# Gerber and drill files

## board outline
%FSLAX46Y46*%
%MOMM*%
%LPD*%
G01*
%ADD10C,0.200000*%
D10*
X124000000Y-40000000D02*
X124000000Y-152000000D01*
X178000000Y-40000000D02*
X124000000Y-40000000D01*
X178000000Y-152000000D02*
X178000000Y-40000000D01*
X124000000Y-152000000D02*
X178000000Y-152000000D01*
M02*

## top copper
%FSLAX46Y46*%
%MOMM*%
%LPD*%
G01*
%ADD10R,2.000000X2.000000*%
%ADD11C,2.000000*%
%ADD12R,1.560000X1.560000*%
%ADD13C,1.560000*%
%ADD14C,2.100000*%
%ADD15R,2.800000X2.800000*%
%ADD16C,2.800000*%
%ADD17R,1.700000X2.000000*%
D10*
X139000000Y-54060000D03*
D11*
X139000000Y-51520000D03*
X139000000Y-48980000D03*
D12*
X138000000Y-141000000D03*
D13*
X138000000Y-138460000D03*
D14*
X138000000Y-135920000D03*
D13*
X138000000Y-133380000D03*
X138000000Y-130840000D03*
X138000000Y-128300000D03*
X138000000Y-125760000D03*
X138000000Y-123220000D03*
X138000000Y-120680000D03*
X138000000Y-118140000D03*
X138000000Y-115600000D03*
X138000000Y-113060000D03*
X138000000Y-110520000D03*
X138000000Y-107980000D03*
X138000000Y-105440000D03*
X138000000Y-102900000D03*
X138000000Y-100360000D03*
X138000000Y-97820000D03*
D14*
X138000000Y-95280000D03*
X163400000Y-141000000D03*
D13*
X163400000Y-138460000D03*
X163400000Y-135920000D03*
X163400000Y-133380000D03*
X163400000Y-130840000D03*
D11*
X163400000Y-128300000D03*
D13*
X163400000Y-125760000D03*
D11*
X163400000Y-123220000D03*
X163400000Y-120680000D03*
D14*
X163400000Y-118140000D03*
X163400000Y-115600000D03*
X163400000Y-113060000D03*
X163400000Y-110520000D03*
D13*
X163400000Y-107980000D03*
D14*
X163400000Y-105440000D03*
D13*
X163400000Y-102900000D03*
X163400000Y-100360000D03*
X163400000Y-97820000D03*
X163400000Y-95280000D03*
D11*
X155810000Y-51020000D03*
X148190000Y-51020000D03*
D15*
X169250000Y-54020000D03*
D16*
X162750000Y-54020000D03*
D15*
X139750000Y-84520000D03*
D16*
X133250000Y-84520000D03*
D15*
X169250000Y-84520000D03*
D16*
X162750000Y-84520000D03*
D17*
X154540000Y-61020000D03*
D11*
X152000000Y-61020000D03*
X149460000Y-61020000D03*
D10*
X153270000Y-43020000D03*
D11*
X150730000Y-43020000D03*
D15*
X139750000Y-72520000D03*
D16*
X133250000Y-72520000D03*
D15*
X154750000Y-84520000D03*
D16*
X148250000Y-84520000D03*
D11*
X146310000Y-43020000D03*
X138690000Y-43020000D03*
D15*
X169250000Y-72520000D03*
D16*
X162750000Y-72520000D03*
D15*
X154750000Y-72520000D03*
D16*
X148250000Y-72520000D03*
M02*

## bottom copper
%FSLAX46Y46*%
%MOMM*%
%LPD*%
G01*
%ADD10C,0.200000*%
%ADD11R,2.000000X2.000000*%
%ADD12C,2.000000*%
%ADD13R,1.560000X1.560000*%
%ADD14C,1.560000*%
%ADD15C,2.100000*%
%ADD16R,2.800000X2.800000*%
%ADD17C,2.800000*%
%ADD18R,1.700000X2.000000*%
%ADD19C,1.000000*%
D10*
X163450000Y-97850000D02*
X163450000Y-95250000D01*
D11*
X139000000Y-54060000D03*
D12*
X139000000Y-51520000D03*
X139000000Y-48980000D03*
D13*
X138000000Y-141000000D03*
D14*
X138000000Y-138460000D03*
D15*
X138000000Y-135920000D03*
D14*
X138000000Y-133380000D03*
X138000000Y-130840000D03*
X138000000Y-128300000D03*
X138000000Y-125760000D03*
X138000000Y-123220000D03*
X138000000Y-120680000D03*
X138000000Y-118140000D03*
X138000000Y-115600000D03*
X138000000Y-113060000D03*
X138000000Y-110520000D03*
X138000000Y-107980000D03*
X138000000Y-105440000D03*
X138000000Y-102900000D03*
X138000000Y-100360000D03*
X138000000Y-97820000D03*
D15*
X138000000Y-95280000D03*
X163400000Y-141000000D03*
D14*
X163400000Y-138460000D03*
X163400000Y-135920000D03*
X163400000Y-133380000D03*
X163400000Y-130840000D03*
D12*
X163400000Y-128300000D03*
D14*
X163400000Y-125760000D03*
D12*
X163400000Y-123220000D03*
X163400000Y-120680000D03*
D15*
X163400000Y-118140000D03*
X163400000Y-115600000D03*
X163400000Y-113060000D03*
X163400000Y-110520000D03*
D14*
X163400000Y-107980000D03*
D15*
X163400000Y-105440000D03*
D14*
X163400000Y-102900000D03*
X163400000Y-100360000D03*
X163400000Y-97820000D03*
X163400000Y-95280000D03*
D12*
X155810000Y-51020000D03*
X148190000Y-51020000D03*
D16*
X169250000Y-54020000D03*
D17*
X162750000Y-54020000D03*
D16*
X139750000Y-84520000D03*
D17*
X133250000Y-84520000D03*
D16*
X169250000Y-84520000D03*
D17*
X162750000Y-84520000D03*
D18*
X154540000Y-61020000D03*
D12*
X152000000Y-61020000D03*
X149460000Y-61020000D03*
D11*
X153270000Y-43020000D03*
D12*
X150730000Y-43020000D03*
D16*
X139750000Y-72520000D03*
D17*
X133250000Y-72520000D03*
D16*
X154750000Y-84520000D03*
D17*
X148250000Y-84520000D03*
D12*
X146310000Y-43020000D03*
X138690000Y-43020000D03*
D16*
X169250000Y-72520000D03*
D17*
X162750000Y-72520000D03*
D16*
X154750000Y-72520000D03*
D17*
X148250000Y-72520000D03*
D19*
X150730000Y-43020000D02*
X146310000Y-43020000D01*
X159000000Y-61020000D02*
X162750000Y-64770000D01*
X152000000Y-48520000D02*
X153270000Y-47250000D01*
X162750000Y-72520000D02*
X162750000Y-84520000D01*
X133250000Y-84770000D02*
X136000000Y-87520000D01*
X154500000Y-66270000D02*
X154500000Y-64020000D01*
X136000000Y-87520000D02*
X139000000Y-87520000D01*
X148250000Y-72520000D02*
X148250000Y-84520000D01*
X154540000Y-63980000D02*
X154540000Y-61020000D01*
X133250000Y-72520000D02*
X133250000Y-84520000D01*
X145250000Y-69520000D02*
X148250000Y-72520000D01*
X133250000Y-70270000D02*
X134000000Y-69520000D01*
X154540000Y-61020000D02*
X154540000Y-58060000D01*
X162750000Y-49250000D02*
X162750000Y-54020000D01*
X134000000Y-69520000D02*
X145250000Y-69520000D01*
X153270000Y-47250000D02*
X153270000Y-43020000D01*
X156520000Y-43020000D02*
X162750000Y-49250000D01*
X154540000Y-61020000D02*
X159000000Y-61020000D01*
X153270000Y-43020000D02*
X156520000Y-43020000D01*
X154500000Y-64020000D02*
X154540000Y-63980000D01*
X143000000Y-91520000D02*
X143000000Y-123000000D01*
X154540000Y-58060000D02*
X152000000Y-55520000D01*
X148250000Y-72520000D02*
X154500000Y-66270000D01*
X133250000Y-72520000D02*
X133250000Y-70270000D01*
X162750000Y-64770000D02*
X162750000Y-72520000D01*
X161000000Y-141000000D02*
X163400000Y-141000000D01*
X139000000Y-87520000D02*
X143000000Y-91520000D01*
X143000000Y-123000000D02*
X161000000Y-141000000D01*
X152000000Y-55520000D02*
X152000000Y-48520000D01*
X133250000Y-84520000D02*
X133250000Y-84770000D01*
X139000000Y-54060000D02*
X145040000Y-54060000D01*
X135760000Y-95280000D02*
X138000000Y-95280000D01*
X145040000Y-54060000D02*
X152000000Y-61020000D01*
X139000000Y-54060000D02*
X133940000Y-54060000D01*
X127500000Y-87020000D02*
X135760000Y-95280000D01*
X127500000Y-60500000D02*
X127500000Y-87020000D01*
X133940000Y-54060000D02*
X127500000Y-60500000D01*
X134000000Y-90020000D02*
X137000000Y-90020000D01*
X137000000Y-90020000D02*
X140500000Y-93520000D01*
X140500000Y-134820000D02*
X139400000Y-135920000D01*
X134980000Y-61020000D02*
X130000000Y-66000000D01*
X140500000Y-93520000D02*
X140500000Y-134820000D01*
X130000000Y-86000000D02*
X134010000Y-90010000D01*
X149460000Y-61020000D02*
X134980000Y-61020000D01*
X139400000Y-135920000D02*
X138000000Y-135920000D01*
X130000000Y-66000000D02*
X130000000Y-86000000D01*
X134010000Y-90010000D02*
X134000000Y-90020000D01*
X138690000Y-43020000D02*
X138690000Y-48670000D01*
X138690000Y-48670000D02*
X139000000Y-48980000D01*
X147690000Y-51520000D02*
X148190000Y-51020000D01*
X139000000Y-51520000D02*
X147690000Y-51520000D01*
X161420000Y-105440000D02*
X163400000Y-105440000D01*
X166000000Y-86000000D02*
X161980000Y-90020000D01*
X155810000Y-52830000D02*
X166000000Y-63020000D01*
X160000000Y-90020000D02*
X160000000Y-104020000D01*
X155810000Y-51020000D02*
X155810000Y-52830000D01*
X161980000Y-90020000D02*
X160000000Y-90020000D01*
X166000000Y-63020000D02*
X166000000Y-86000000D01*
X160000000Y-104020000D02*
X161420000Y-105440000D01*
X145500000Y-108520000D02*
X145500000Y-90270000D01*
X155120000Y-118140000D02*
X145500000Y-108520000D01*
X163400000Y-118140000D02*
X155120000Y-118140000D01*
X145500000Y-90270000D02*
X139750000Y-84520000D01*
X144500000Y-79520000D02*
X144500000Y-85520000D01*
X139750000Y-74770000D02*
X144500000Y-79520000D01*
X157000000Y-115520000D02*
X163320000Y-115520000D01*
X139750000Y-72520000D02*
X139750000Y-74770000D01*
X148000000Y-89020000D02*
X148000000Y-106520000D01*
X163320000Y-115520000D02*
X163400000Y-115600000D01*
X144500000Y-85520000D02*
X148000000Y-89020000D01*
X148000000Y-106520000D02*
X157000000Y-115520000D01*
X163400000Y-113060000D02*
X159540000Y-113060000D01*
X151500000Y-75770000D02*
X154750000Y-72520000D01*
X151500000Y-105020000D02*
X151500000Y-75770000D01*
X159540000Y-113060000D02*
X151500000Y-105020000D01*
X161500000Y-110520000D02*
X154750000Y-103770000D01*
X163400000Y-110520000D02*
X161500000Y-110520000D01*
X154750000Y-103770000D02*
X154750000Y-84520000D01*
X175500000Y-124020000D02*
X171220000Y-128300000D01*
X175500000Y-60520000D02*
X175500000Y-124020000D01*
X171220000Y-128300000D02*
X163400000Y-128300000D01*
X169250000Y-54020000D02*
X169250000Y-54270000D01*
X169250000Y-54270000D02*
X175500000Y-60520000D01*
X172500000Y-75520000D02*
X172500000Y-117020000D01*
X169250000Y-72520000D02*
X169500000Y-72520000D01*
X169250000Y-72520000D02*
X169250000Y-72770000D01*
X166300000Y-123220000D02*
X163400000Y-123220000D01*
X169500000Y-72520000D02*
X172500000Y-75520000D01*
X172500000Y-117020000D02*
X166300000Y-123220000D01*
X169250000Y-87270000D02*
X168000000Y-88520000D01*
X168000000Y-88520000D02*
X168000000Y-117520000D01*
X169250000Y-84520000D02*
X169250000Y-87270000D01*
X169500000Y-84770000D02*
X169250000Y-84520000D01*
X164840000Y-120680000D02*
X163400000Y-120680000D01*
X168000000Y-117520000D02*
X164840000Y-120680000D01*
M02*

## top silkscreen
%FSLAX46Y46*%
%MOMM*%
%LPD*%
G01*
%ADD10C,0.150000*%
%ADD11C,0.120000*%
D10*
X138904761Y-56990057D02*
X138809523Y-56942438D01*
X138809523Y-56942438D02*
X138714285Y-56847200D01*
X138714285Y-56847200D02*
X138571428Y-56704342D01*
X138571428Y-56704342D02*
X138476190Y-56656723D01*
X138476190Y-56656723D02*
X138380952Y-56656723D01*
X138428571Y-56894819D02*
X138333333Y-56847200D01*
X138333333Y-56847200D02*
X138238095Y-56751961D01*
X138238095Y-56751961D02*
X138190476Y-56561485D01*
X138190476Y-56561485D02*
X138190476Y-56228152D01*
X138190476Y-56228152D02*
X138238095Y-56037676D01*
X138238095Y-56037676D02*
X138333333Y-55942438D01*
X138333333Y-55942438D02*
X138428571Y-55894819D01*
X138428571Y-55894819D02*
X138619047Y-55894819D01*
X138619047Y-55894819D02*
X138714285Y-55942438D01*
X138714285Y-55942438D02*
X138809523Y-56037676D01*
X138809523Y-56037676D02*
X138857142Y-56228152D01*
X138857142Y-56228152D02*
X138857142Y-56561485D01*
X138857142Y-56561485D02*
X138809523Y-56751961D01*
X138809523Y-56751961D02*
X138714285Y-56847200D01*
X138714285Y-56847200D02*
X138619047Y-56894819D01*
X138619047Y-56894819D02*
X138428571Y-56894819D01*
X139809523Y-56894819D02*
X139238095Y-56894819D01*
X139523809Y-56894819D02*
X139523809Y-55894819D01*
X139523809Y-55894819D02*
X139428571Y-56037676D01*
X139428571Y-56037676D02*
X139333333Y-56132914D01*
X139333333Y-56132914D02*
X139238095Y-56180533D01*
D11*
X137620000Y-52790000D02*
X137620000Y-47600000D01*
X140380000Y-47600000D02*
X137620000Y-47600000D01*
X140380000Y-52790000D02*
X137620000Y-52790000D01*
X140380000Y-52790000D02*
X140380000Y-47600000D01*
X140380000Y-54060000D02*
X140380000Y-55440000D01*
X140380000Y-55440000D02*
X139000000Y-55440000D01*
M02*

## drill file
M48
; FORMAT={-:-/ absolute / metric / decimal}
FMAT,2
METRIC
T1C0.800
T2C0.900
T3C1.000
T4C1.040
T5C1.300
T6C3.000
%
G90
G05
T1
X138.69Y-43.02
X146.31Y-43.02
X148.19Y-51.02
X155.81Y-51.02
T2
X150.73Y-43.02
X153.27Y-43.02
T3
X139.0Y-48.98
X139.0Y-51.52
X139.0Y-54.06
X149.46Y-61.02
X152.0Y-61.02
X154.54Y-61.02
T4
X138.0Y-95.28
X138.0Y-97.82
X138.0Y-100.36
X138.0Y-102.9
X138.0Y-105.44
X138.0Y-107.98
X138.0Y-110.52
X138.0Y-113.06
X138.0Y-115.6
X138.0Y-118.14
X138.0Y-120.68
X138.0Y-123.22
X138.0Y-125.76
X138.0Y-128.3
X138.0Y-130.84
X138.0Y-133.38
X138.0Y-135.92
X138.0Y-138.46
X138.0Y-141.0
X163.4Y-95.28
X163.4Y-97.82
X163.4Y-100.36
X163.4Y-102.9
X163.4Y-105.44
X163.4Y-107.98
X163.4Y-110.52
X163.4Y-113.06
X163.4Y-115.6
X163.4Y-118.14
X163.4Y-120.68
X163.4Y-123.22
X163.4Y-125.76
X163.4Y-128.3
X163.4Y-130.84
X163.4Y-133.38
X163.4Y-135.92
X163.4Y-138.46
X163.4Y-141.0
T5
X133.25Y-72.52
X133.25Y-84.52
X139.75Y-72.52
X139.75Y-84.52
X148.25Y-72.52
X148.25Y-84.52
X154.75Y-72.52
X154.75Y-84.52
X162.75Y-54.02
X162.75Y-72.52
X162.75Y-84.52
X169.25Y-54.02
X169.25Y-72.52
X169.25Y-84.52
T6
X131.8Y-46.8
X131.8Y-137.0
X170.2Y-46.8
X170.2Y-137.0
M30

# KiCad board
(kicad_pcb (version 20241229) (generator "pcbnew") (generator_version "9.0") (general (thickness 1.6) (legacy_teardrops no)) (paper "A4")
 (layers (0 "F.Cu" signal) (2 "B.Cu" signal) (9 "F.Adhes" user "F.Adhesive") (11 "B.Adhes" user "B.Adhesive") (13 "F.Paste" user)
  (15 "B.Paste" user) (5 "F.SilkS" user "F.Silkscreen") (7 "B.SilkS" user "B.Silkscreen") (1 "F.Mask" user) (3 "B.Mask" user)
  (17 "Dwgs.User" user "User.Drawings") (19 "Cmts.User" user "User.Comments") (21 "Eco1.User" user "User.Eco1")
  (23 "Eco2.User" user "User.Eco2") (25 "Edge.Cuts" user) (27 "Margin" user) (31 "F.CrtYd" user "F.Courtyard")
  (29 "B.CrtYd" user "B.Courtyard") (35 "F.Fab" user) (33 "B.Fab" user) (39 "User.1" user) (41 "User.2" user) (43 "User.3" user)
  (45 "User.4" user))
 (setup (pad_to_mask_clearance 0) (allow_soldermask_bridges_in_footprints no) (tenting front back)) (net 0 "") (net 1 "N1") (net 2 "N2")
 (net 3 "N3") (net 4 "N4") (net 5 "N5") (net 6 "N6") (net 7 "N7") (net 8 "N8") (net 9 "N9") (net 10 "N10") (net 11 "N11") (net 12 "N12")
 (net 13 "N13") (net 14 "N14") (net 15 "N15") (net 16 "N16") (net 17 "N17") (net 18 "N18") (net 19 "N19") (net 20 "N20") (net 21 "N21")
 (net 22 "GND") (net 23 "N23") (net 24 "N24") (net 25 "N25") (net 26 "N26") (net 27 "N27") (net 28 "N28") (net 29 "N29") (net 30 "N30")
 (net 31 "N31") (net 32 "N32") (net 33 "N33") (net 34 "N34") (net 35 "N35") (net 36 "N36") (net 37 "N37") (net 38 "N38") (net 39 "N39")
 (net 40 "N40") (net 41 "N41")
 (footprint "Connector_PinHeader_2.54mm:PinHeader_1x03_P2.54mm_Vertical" (layer "F.Cu") (at 139 54.06 180)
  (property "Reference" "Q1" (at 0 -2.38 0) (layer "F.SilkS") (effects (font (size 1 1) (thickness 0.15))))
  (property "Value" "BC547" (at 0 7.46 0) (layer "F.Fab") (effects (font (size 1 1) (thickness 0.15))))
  (fp_line (start 1.38 1.27) (end 1.38 6.46) (stroke (width 0.12) (type solid)) (layer "F.SilkS"))
  (fp_line (start -1.38 6.46) (end 1.38 6.46) (stroke (width 0.12) (type solid)) (layer "F.SilkS"))
  (fp_line (start -1.38 1.27) (end 1.38 1.27) (stroke (width 0.12) (type solid)) (layer "F.SilkS"))
  (fp_line (start -1.38 1.27) (end -1.38 6.46) (stroke (width 0.12) (type solid)) (layer "F.SilkS"))
  (fp_line (start -1.38 0) (end -1.38 -1.38) (stroke (width 0.12) (type solid)) (layer "F.SilkS"))
  (fp_line (start -1.38 -1.38) (end 0 -1.38) (stroke (width 0.12) (type solid)) (layer "F.SilkS"))
  (pad "1" thru_hole rect (at 0 0 180) (size 2 2) (drill 1) (layers "*.Cu" "*.Mask") (remove_unused_layers no) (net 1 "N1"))
  (pad "2" thru_hole circle (at 0 2.54 180) (size 2 2) (drill 1) (layers "*.Cu" "*.Mask") (remove_unused_layers no) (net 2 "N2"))
  (pad "3" thru_hole circle (at 0 5.08 180) (size 2 2) (drill 1) (layers "*.Cu" "*.Mask") (remove_unused_layers no) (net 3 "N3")))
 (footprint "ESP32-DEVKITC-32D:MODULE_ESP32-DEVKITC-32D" (layer "B.Cu") (at 150.7 121.24)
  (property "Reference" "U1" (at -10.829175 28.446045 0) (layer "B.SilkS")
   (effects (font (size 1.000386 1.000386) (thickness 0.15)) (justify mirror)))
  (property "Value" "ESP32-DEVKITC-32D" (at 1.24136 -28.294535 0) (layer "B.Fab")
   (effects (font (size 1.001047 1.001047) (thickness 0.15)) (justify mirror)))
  (pad "J2-1" thru_hole rect (at -12.7 19.76) (size 1.56 1.56) (drill 1.04) (layers "*.Cu" "*.Mask") (remove_unused_layers no) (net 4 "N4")
   (solder_mask_margin 0.102))
  (pad "J2-2" thru_hole circle (at -12.7 17.22) (size 1.56 1.56) (drill 1.04) (layers "*.Cu" "*.Mask") (remove_unused_layers no)
   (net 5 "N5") (solder_mask_margin 0.102))
  (pad "J2-3" thru_hole circle (at -12.7 14.68) (size 2.1 2.1) (drill 1.04) (layers "*.Cu" "*.Mask") (remove_unused_layers no) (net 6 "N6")
   (solder_mask_margin 0.102))
  (pad "J2-4" thru_hole circle (at -12.7 12.14) (size 1.56 1.56) (drill 1.04) (layers "*.Cu" "*.Mask") (remove_unused_layers no)
   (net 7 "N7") (solder_mask_margin 0.102))
  (pad "J2-5" thru_hole circle (at -12.7 9.6) (size 1.56 1.56) (drill 1.04) (layers "*.Cu" "*.Mask") (remove_unused_layers no) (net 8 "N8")
   (solder_mask_margin 0.102))
  (pad "J2-6" thru_hole circle (at -12.7 7.06) (size 1.56 1.56) (drill 1.04) (layers "*.Cu" "*.Mask") (remove_unused_layers no) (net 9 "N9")
   (solder_mask_margin 0.102))
  (pad "J2-7" thru_hole circle (at -12.7 4.52) (size 1.56 1.56) (drill 1.04) (layers "*.Cu" "*.Mask") (remove_unused_layers no)
   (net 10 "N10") (solder_mask_margin 0.102))
  (pad "J2-8" thru_hole circle (at -12.7 1.98) (size 1.56 1.56) (drill 1.04) (layers "*.Cu" "*.Mask") (remove_unused_layers no)
   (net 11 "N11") (solder_mask_margin 0.102))
  (pad "J2-9" thru_hole circle (at -12.7 -0.56) (size 1.56 1.56) (drill 1.04) (layers "*.Cu" "*.Mask") (remove_unused_layers no)
   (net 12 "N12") (solder_mask_margin 0.102))
  (pad "J2-10" thru_hole circle (at -12.7 -3.1) (size 1.56 1.56) (drill 1.04) (layers "*.Cu" "*.Mask") (remove_unused_layers no)
   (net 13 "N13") (solder_mask_margin 0.102))
  (pad "J2-11" thru_hole circle (at -12.7 -5.64) (size 1.56 1.56) (drill 1.04) (layers "*.Cu" "*.Mask") (remove_unused_layers no)
   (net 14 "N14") (solder_mask_margin 0.102))
  (pad "J2-12" thru_hole circle (at -12.7 -8.18) (size 1.56 1.56) (drill 1.04) (layers "*.Cu" "*.Mask") (remove_unused_layers no)
   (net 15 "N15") (solder_mask_margin 0.102))
  (pad "J2-13" thru_hole circle (at -12.7 -10.72) (size 1.56 1.56) (drill 1.04) (layers "*.Cu" "*.Mask") (remove_unused_layers no)
   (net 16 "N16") (solder_mask_margin 0.102))
  (pad "J2-14" thru_hole circle (at -12.7 -13.26) (size 1.56 1.56) (drill 1.04) (layers "*.Cu" "*.Mask") (remove_unused_layers no)
   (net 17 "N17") (solder_mask_margin 0.102))
  (pad "J2-15" thru_hole circle (at -12.7 -15.8) (size 1.56 1.56) (drill 1.04) (layers "*.Cu" "*.Mask") (remove_unused_layers no)
   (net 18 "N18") (solder_mask_margin 0.102))
  (pad "J2-16" thru_hole circle (at -12.7 -18.34) (size 1.56 1.56) (drill 1.04) (layers "*.Cu" "*.Mask") (remove_unused_layers no)
   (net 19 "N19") (solder_mask_margin 0.102))
  (pad "J2-17" thru_hole circle (at -12.7 -20.88) (size 1.56 1.56) (drill 1.04) (layers "*.Cu" "*.Mask") (remove_unused_layers no)
   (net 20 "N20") (solder_mask_margin 0.102))
  (pad "J2-18" thru_hole circle (at -12.7 -23.42) (size 1.56 1.56) (drill 1.04) (layers "*.Cu" "*.Mask") (remove_unused_layers no)
   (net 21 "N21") (solder_mask_margin 0.102))
  (pad "J2-19" thru_hole circle (at -12.7 -25.96) (size 2.1 2.1) (drill 1.04) (layers "*.Cu" "*.Mask") (remove_unused_layers no)
   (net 1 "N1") (solder_mask_margin 0.102))
  (pad "J3-1" thru_hole circle (at 12.7 19.76) (size 2.1 2.1) (drill 1.04) (layers "*.Cu" "*.Mask") (remove_unused_layers no) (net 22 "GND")
   (solder_mask_margin 0.102))
  (pad "J3-2" thru_hole circle (at 12.7 17.22) (size 1.56 1.56) (drill 1.04) (layers "*.Cu" "*.Mask") (remove_unused_layers no)
   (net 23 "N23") (solder_mask_margin 0.102))
  (pad "J3-3" thru_hole circle (at 12.7 14.68) (size 1.56 1.56) (drill 1.04) (layers "*.Cu" "*.Mask") (remove_unused_layers no)
   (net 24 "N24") (solder_mask_margin 0.102))
  (pad "J3-4" thru_hole circle (at 12.7 12.14) (size 1.56 1.56) (drill 1.04) (layers "*.Cu" "*.Mask") (remove_unused_layers no)
   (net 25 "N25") (solder_mask_margin 0.102))
  (pad "J3-5" thru_hole circle (at 12.7 9.6) (size 1.56 1.56) (drill 1.04) (layers "*.Cu" "*.Mask") (remove_unused_layers no) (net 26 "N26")
   (solder_mask_margin 0.102))
  (pad "J3-6" thru_hole circle (at 12.7 7.06) (size 2 2) (drill 1.04) (layers "*.Cu" "*.Mask") (remove_unused_layers no) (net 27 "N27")
   (solder_mask_margin 0.102))
  (pad "J3-7" thru_hole circle (at 12.7 4.52) (size 1.56 1.56) (drill 1.04) (layers "*.Cu" "*.Mask") (remove_unused_layers no)
   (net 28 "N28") (solder_mask_margin 0.102))
  (pad "J3-8" thru_hole circle (at 12.7 1.98) (size 2 2) (drill 1.04) (layers "*.Cu" "*.Mask") (remove_unused_layers no) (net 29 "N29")
   (solder_mask_margin 0.102))
  (pad "J3-9" thru_hole circle (at 12.7 -0.56) (size 2 2) (drill 1.04) (layers "*.Cu" "*.Mask") (remove_unused_layers no) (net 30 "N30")
   (solder_mask_margin 0.102))
  (pad "J3-10" thru_hole circle (at 12.7 -3.1) (size 2.1 2.1) (drill 1.04) (layers "*.Cu" "*.Mask") (remove_unused_layers no) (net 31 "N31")
   (solder_mask_margin 0.102))
  (pad "J3-11" thru_hole circle (at 12.7 -5.64) (size 2.1 2.1) (drill 1.04) (layers "*.Cu" "*.Mask") (remove_unused_layers no)
   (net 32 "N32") (solder_mask_margin 0.102))
  (pad "J3-12" thru_hole circle (at 12.7 -8.18) (size 2.1 2.1) (drill 1.04) (layers "*.Cu" "*.Mask") (remove_unused_layers no)
   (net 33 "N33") (solder_mask_margin 0.102))
  (pad "J3-13" thru_hole circle (at 12.7 -10.72) (size 2.1 2.1) (drill 1.04) (layers "*.Cu" "*.Mask") (remove_unused_layers no)
   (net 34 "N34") (solder_mask_margin 0.102))
  (pad "J3-14" thru_hole circle (at 12.7 -13.26) (size 1.56 1.56) (drill 1.04) (layers "*.Cu" "*.Mask") (remove_unused_layers no)
   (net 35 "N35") (solder_mask_margin 0.102))
  (pad "J3-15" thru_hole circle (at 12.7 -15.8) (size 2.1 2.1) (drill 1.04) (layers "*.Cu" "*.Mask") (remove_unused_layers no)
   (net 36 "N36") (solder_mask_margin 0.102))
  (pad "J3-16" thru_hole circle (at 12.7 -18.34) (size 1.56 1.56) (drill 1.04) (layers "*.Cu" "*.Mask") (remove_unused_layers no)
   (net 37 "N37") (solder_mask_margin 0.102))
  (pad "J3-17" thru_hole circle (at 12.7 -20.88) (size 1.56 1.56) (drill 1.04) (layers "*.Cu" "*.Mask") (remove_unused_layers no)
   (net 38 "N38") (solder_mask_margin 0.102))
  (pad "J3-18" thru_hole circle (at 12.7 -23.42) (size 1.56 1.56) (drill 1.04) (layers "*.Cu" "*.Mask") (remove_unused_layers no)
   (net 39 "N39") (solder_mask_margin 0.102))
  (pad "J3-19" thru_hole circle (at 12.7 -25.96) (size 1.56 1.56) (drill 1.04) (layers "*.Cu" "*.Mask") (remove_unused_layers no)
   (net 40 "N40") (solder_mask_margin 0.102)))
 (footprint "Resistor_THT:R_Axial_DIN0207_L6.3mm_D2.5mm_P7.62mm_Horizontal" (layer "B.Cu") (at 155.81 51.02 180)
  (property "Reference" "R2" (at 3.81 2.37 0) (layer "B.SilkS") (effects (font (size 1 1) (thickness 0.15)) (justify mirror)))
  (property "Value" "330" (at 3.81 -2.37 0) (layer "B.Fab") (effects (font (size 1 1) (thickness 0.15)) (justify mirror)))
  (pad "1" thru_hole circle (at 0 0 180) (size 2 2) (drill 0.8) (layers "*.Cu" "*.Mask") (remove_unused_layers no) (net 36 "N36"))
  (pad "2" thru_hole circle (at 7.62 0 180) (size 2 2) (drill 0.8) (layers "*.Cu" "*.Mask") (remove_unused_layers no) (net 2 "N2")))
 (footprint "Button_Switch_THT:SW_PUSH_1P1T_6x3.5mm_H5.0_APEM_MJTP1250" (layer "B.Cu") (at 169.25 54.02 180)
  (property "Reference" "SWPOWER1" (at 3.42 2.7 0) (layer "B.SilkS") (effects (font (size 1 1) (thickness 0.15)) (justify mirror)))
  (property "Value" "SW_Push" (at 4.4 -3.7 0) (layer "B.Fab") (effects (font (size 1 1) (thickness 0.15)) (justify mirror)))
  (pad "1" thru_hole rect (at 0 0 90) (size 2.8 2.8) (drill 1.3) (layers "*.Cu" "*.Mask") (remove_unused_layers no) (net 27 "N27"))
  (pad "2" thru_hole circle (at 6.5 0 90) (size 2.8 2.8) (drill 1.3) (layers "*.Cu" "*.Mask") (remove_unused_layers no) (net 22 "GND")))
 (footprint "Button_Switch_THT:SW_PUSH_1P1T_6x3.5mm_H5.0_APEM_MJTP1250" (layer "B.Cu") (at 139.75 84.52 180)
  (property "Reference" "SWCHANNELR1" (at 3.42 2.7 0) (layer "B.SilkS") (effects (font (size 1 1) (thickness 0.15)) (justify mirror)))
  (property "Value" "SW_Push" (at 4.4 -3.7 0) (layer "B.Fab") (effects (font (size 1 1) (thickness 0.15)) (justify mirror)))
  (pad "1" thru_hole rect (at 0 0 90) (size 2.8 2.8) (drill 1.3) (layers "*.Cu" "*.Mask") (remove_unused_layers no) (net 31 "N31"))
  (pad "2" thru_hole circle (at 6.5 0 90) (size 2.8 2.8) (drill 1.3) (layers "*.Cu" "*.Mask") (remove_unused_layers no) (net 22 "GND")))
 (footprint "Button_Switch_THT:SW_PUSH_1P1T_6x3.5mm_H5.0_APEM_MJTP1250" (layer "B.Cu") (at 169.25 84.52 180)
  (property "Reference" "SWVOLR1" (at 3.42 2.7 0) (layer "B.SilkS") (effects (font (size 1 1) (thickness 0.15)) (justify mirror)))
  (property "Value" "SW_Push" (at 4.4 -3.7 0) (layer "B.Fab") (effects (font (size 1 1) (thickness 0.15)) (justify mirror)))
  (pad "1" thru_hole rect (at 0 0 90) (size 2.8 2.8) (drill 1.3) (layers "*.Cu" "*.Mask") (remove_unused_layers no) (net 30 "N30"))
  (pad "2" thru_hole circle (at 6.5 0 90) (size 2.8 2.8) (drill 1.3) (layers "*.Cu" "*.Mask") (remove_unused_layers no) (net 22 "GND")))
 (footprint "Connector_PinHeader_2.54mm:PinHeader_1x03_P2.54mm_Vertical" (layer "B.Cu") (at 154.54 61.02 90)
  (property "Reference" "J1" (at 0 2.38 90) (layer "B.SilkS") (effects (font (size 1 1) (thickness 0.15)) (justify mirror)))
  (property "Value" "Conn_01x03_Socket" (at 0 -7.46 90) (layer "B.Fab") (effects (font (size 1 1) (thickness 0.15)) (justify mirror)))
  (pad "1" thru_hole rect (at 0 0 90) (size 2 1.7) (drill 1) (layers "*.Cu" "*.Mask") (remove_unused_layers no) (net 22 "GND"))
  (pad "2" thru_hole circle (at 0 -2.54 90) (size 2 2) (drill 1) (layers "*.Cu" "*.Mask") (remove_unused_layers no) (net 1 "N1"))
  (pad "3" thru_hole circle (at 0 -5.08 90) (size 2 2) (drill 1) (layers "*.Cu" "*.Mask") (remove_unused_layers no) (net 6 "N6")))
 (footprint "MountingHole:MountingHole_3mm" (layer "B.Cu") (at 131.8 137 180)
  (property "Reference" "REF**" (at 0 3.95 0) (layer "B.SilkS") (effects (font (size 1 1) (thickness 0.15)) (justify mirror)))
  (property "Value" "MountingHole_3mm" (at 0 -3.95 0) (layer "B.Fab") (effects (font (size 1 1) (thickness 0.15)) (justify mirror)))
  (pad "" np_thru_hole circle (at 0 0 180) (size 3 3) (drill 3) (layers "*.Cu" "*.Mask")))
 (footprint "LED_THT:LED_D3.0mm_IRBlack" (layer "B.Cu") (at 153.27 43.02 180)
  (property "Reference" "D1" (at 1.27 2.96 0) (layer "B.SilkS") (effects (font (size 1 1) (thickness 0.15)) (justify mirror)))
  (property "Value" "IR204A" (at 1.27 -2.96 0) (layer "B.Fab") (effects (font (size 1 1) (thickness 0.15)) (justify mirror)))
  (pad "1" thru_hole rect (at 0 0 180) (size 2 2) (drill 0.9) (layers "*.Cu" "*.Mask") (remove_unused_layers no) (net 22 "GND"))
  (pad "2" thru_hole circle (at 2.54 0 180) (size 2 2) (drill 0.9) (layers "*.Cu" "*.Mask") (remove_unused_layers no) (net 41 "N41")))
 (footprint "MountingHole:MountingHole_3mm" (layer "B.Cu") (at 131.8 46.8 180)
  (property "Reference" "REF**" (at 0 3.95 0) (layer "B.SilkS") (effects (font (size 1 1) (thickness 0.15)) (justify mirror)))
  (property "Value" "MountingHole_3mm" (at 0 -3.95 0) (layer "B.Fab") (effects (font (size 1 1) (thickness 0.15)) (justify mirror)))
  (pad "" np_thru_hole circle (at 0 0 180) (size 3 3) (drill 3) (layers "*.Cu" "*.Mask")))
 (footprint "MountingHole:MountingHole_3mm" (layer "B.Cu") (at 170.2 137 180)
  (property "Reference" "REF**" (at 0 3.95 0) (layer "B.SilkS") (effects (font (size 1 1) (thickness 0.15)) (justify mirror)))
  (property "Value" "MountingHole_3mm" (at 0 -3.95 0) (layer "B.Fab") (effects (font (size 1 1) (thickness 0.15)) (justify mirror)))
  (pad "" np_thru_hole circle (at 0 0 180) (size 3 3) (drill 3) (layers "*.Cu" "*.Mask")))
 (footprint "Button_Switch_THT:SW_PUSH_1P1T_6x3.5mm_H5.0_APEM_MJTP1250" (layer "B.Cu") (at 139.75 72.52 180)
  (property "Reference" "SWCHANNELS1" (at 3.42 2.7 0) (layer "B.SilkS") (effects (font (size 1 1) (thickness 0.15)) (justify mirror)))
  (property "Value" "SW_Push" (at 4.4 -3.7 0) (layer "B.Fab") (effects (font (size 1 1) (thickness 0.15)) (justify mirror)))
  (pad "1" thru_hole rect (at 0 0 90) (size 2.8 2.8) (drill 1.3) (layers "*.Cu" "*.Mask") (remove_unused_layers no) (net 32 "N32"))
  (pad "2" thru_hole circle (at 6.5 0 90) (size 2.8 2.8) (drill 1.3) (layers "*.Cu" "*.Mask") (remove_unused_layers no) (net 22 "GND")))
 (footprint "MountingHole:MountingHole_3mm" (layer "B.Cu") (at 170.2 46.8 180)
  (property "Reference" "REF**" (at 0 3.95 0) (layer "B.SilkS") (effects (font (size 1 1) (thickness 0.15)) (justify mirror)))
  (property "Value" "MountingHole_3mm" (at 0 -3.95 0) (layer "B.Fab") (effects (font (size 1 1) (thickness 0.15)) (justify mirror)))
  (pad "" np_thru_hole circle (at 0 0 180) (size 3 3) (drill 3) (layers "*.Cu" "*.Mask")))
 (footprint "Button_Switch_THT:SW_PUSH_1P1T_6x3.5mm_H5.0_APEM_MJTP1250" (layer "B.Cu") (at 154.75 84.52 180)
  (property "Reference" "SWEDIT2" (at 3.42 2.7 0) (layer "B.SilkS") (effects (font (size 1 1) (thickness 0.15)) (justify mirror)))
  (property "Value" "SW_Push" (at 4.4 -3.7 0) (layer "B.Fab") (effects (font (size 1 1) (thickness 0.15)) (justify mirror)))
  (pad "1" thru_hole rect (at 0 0 90) (size 2.8 2.8) (drill 1.3) (layers "*.Cu" "*.Mask") (remove_unused_layers no) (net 34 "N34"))
  (pad "2" thru_hole circle (at 6.5 0 90) (size 2.8 2.8) (drill 1.3) (layers "*.Cu" "*.Mask") (remove_unused_layers no) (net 22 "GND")))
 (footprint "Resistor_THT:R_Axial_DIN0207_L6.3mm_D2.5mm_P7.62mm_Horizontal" (layer "B.Cu") (at 146.31 43.02 180)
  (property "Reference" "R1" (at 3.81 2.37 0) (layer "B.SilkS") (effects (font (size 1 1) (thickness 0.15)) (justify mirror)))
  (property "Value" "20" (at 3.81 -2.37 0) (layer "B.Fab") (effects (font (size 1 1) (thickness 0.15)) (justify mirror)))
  (pad "1" thru_hole circle (at 0 0 180) (size 2 2) (drill 0.8) (layers "*.Cu" "*.Mask") (remove_unused_layers no) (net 41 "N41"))
  (pad "2" thru_hole circle (at 7.62 0 180) (size 2 2) (drill 0.8) (layers "*.Cu" "*.Mask") (remove_unused_layers no) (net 3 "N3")))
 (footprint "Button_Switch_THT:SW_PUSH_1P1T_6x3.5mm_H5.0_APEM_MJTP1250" (layer "B.Cu") (at 169.25 72.52 180)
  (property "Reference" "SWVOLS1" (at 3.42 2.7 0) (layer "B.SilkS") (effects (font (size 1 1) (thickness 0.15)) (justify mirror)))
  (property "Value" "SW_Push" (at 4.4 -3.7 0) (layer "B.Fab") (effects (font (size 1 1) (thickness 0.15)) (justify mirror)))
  (pad "1" thru_hole rect (at 0 0 90) (size 2.8 2.8) (drill 1.3) (layers "*.Cu" "*.Mask") (remove_unused_layers no) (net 29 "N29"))
  (pad "2" thru_hole circle (at 6.5 0 90) (size 2.8 2.8) (drill 1.3) (layers "*.Cu" "*.Mask") (remove_unused_layers no) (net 22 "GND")))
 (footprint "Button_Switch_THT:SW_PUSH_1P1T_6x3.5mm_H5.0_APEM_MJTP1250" (layer "B.Cu") (at 154.75 72.52 180)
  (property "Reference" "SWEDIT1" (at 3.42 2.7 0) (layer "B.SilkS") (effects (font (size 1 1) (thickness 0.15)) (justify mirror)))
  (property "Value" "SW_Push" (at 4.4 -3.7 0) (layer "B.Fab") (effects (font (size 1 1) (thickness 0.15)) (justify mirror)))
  (pad "1" thru_hole rect (at 0 0 90) (size 2.8 2.8) (drill 1.3) (layers "*.Cu" "*.Mask") (remove_unused_layers no) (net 33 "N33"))
  (pad "2" thru_hole circle (at 6.5 0 90) (size 2.8 2.8) (drill 1.3) (layers "*.Cu" "*.Mask") (remove_unused_layers no) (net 22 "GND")))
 (gr_line (start 163.45 97.85) (end 163.45 95.25) (stroke (width 0.2) (type default)) (layer "B.Cu"))
 (gr_line (start 124 40) (end 124 152) (stroke (width 0.2) (type solid)) (layer "Edge.Cuts"))
 (gr_line (start 178 40) (end 124 40) (stroke (width 0.2) (type solid)) (layer "Edge.Cuts"))
 (gr_line (start 178 152) (end 178 40) (stroke (width 0.2) (type solid)) (layer "Edge.Cuts"))
 (gr_line (start 124 152) (end 178 152) (stroke (width 0.2) (type solid)) (layer "Edge.Cuts"))
 (segment (start 150.73 43.02) (end 146.31 43.02) (width 1) (layer "B.Cu") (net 41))
 (segment (start 159 61.02) (end 162.75 64.77) (width 1) (layer "B.Cu") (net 22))
 (segment (start 152 48.52) (end 153.27 47.25) (width 1) (layer "B.Cu") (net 22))
 (segment (start 162.75 72.52) (end 162.75 84.52) (width 1) (layer "B.Cu") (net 22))
 (segment (start 133.25 84.77) (end 136 87.52) (width 1) (layer "B.Cu") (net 22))
 (segment (start 154.5 66.27) (end 154.5 64.02) (width 1) (layer "B.Cu") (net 22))
 (segment (start 136 87.52) (end 139 87.52) (width 1) (layer "B.Cu") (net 22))
 (segment (start 148.25 72.52) (end 148.25 84.52) (width 1) (layer "B.Cu") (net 22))
 (segment (start 154.54 63.98) (end 154.54 61.02) (width 1) (layer "B.Cu") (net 22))
 (segment (start 133.25 72.52) (end 133.25 84.52) (width 1) (layer "B.Cu") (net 22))
 (segment (start 145.25 69.52) (end 148.25 72.52) (width 1) (layer "B.Cu") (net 22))
 (segment (start 133.25 70.27) (end 134 69.52) (width 1) (layer "B.Cu") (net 22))
 (segment (start 154.54 61.02) (end 154.54 58.06) (width 1) (layer "B.Cu") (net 22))
 (segment (start 162.75 49.25) (end 162.75 54.02) (width 1) (layer "B.Cu") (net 22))
 (segment (start 134 69.52) (end 145.25 69.52) (width 1) (layer "B.Cu") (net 22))
 (segment (start 153.27 47.25) (end 153.27 43.02) (width 1) (layer "B.Cu") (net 22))
 (segment (start 156.52 43.02) (end 162.75 49.25) (width 1) (layer "B.Cu") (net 22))
 (segment (start 154.54 61.02) (end 159 61.02) (width 1) (layer "B.Cu") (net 22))
 (segment (start 153.27 43.02) (end 156.52 43.02) (width 1) (layer "B.Cu") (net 22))
 (segment (start 154.5 64.02) (end 154.54 63.98) (width 1) (layer "B.Cu") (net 22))
 (segment (start 143 91.52) (end 143 123) (width 1) (layer "B.Cu") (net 22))
 (segment (start 154.54 58.06) (end 152 55.52) (width 1) (layer "B.Cu") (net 22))
 (segment (start 148.25 72.52) (end 154.5 66.27) (width 1) (layer "B.Cu") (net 22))
 (segment (start 133.25 72.52) (end 133.25 70.27) (width 1) (layer "B.Cu") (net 22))
 (segment (start 162.75 64.77) (end 162.75 72.52) (width 1) (layer "B.Cu") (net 22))
 (segment (start 161 141) (end 163.4 141) (width 1) (layer "B.Cu") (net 22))
 (segment (start 139 87.52) (end 143 91.52) (width 1) (layer "B.Cu") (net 22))
 (segment (start 143 123) (end 161 141) (width 1) (layer "B.Cu") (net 22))
 (segment (start 152 55.52) (end 152 48.52) (width 1) (layer "B.Cu") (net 22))
 (segment (start 133.25 84.52) (end 133.25 84.77) (width 1) (layer "B.Cu") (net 22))
 (segment (start 139 54.06) (end 145.04 54.06) (width 1) (layer "B.Cu") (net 1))
 (segment (start 135.76 95.28) (end 138 95.28) (width 1) (layer "B.Cu") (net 1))
 (segment (start 145.04 54.06) (end 152 61.02) (width 1) (layer "B.Cu") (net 1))
 (segment (start 139 54.06) (end 133.94 54.06) (width 1) (layer "B.Cu") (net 1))
 (segment (start 127.5 87.02) (end 135.76 95.28) (width 1) (layer "B.Cu") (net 1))
 (segment (start 127.5 60.5) (end 127.5 87.02) (width 1) (layer "B.Cu") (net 1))
 (segment (start 133.94 54.06) (end 127.5 60.5) (width 1) (layer "B.Cu") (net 1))
 (segment (start 134 90.02) (end 137 90.02) (width 1) (layer "B.Cu") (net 6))
 (segment (start 137 90.02) (end 140.5 93.52) (width 1) (layer "B.Cu") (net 6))
 (segment (start 140.5 134.82) (end 139.4 135.92) (width 1) (layer "B.Cu") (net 6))
 (segment (start 134.98 61.02) (end 130 66) (width 1) (layer "B.Cu") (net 6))
 (segment (start 140.5 93.52) (end 140.5 134.82) (width 1) (layer "B.Cu") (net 6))
 (segment (start 130 86) (end 134.01 90.01) (width 1) (layer "B.Cu") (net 6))
 (segment (start 149.46 61.02) (end 134.98 61.02) (width 1) (layer "B.Cu") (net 6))
 (segment (start 139.4 135.92) (end 138 135.92) (width 1) (layer "B.Cu") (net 6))
 (segment (start 130 66) (end 130 86) (width 1) (layer "B.Cu") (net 6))
 (segment (start 134.01 90.01) (end 134 90.02) (width 1) (layer "B.Cu") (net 6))
 (segment (start 138.69 43.02) (end 138.69 48.67) (width 1) (layer "B.Cu") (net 3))
 (segment (start 138.69 48.67) (end 139 48.98) (width 1) (layer "B.Cu") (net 3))
 (segment (start 147.69 51.52) (end 148.19 51.02) (width 1) (layer "B.Cu") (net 2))
 (segment (start 139 51.52) (end 147.69 51.52) (width 1) (layer "B.Cu") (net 2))
 (segment (start 161.42 105.44) (end 163.4 105.44) (width 1) (layer "B.Cu") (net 36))
 (segment (start 166 86) (end 161.98 90.02) (width 1) (layer "B.Cu") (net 36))
 (segment (start 155.81 52.83) (end 166 63.02) (width 1) (layer "B.Cu") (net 36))
 (segment (start 160 90.02) (end 160 104.02) (width 1) (layer "B.Cu") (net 36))
 (segment (start 155.81 51.02) (end 155.81 52.83) (width 1) (layer "B.Cu") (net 36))
 (segment (start 161.98 90.02) (end 160 90.02) (width 1) (layer "B.Cu") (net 36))
 (segment (start 166 63.02) (end 166 86) (width 1) (layer "B.Cu") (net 36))
 (segment (start 160 104.02) (end 161.42 105.44) (width 1) (layer "B.Cu") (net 36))
 (segment (start 145.5 108.52) (end 145.5 90.27) (width 1) (layer "B.Cu") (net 31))
 (segment (start 155.12 118.14) (end 145.5 108.52) (width 1) (layer "B.Cu") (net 31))
 (segment (start 163.4 118.14) (end 155.12 118.14) (width 1) (layer "B.Cu") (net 31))
 (segment (start 145.5 90.27) (end 139.75 84.52) (width 1) (layer "B.Cu") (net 31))
 (segment (start 144.5 79.52) (end 144.5 85.52) (width 1) (layer "B.Cu") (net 32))
 (segment (start 139.75 74.77) (end 144.5 79.52) (width 1) (layer "B.Cu") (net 32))
 (segment (start 157 115.52) (end 163.32 115.52) (width 1) (layer "B.Cu") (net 32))
 (segment (start 139.75 72.52) (end 139.75 74.77) (width 1) (layer "B.Cu") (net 32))
 (segment (start 148 89.02) (end 148 106.52) (width 1) (layer "B.Cu") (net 32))
 (segment (start 163.32 115.52) (end 163.4 115.6) (width 1) (layer "B.Cu") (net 32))
 (segment (start 144.5 85.52) (end 148 89.02) (width 1) (layer "B.Cu") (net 32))
 (segment (start 148 106.52) (end 157 115.52) (width 1) (layer "B.Cu") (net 32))
 (segment (start 163.4 113.06) (end 159.54 113.06) (width 1) (layer "B.Cu") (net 33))
 (segment (start 151.5 75.77) (end 154.75 72.52) (width 1) (layer "B.Cu") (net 33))
 (segment (start 151.5 105.02) (end 151.5 75.77) (width 1) (layer "B.Cu") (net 33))
 (segment (start 159.54 113.06) (end 151.5 105.02) (width 1) (layer "B.Cu") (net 33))
 (segment (start 161.5 110.52) (end 154.75 103.77) (width 1) (layer "B.Cu") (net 34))
 (segment (start 163.4 110.52) (end 161.5 110.52) (width 1) (layer "B.Cu") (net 34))
 (segment (start 154.75 103.77) (end 154.75 84.52) (width 1) (layer "B.Cu") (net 34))
 (segment (start 175.5 124.02) (end 171.22 128.3) (width 1) (layer "B.Cu") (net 27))
 (segment (start 175.5 60.52) (end 175.5 124.02) (width 1) (layer "B.Cu") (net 27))
 (segment (start 171.22 128.3) (end 163.4 128.3) (width 1) (layer "B.Cu") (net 27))
 (segment (start 169.25 54.02) (end 169.25 54.27) (width 1) (layer "B.Cu") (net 27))
 (segment (start 169.25 54.27) (end 175.5 60.52) (width 1) (layer "B.Cu") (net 27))
 (segment (start 172.5 75.52) (end 172.5 117.02) (width 1) (layer "B.Cu") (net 29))
 (segment (start 169.25 72.52) (end 169.5 72.52) (width 1) (layer "B.Cu") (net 29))
 (segment (start 169.25 72.52) (end 169.25 72.77) (width 1) (layer "B.Cu") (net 29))
 (segment (start 166.3 123.22) (end 163.4 123.22) (width 1) (layer "B.Cu") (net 29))
 (segment (start 169.5 72.52) (end 172.5 75.52) (width 1) (layer "B.Cu") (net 29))
 (segment (start 172.5 117.02) (end 166.3 123.22) (width 1) (layer "B.Cu") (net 29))
 (segment (start 169.25 87.27) (end 168 88.52) (width 1) (layer "B.Cu") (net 30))
 (segment (start 168 88.52) (end 168 117.52) (width 1) (layer "B.Cu") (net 30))
 (segment (start 169.25 84.52) (end 169.25 87.27) (width 1) (layer "B.Cu") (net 30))
 (segment (start 169.5 84.77) (end 169.25 84.52) (width 1) (layer "B.Cu") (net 30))
 (segment (start 164.84 120.68) (end 163.4 120.68) (width 1) (layer "B.Cu") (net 30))
 (segment (start 168 117.52) (end 164.84 120.68) (width 1) (layer "B.Cu") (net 30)))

